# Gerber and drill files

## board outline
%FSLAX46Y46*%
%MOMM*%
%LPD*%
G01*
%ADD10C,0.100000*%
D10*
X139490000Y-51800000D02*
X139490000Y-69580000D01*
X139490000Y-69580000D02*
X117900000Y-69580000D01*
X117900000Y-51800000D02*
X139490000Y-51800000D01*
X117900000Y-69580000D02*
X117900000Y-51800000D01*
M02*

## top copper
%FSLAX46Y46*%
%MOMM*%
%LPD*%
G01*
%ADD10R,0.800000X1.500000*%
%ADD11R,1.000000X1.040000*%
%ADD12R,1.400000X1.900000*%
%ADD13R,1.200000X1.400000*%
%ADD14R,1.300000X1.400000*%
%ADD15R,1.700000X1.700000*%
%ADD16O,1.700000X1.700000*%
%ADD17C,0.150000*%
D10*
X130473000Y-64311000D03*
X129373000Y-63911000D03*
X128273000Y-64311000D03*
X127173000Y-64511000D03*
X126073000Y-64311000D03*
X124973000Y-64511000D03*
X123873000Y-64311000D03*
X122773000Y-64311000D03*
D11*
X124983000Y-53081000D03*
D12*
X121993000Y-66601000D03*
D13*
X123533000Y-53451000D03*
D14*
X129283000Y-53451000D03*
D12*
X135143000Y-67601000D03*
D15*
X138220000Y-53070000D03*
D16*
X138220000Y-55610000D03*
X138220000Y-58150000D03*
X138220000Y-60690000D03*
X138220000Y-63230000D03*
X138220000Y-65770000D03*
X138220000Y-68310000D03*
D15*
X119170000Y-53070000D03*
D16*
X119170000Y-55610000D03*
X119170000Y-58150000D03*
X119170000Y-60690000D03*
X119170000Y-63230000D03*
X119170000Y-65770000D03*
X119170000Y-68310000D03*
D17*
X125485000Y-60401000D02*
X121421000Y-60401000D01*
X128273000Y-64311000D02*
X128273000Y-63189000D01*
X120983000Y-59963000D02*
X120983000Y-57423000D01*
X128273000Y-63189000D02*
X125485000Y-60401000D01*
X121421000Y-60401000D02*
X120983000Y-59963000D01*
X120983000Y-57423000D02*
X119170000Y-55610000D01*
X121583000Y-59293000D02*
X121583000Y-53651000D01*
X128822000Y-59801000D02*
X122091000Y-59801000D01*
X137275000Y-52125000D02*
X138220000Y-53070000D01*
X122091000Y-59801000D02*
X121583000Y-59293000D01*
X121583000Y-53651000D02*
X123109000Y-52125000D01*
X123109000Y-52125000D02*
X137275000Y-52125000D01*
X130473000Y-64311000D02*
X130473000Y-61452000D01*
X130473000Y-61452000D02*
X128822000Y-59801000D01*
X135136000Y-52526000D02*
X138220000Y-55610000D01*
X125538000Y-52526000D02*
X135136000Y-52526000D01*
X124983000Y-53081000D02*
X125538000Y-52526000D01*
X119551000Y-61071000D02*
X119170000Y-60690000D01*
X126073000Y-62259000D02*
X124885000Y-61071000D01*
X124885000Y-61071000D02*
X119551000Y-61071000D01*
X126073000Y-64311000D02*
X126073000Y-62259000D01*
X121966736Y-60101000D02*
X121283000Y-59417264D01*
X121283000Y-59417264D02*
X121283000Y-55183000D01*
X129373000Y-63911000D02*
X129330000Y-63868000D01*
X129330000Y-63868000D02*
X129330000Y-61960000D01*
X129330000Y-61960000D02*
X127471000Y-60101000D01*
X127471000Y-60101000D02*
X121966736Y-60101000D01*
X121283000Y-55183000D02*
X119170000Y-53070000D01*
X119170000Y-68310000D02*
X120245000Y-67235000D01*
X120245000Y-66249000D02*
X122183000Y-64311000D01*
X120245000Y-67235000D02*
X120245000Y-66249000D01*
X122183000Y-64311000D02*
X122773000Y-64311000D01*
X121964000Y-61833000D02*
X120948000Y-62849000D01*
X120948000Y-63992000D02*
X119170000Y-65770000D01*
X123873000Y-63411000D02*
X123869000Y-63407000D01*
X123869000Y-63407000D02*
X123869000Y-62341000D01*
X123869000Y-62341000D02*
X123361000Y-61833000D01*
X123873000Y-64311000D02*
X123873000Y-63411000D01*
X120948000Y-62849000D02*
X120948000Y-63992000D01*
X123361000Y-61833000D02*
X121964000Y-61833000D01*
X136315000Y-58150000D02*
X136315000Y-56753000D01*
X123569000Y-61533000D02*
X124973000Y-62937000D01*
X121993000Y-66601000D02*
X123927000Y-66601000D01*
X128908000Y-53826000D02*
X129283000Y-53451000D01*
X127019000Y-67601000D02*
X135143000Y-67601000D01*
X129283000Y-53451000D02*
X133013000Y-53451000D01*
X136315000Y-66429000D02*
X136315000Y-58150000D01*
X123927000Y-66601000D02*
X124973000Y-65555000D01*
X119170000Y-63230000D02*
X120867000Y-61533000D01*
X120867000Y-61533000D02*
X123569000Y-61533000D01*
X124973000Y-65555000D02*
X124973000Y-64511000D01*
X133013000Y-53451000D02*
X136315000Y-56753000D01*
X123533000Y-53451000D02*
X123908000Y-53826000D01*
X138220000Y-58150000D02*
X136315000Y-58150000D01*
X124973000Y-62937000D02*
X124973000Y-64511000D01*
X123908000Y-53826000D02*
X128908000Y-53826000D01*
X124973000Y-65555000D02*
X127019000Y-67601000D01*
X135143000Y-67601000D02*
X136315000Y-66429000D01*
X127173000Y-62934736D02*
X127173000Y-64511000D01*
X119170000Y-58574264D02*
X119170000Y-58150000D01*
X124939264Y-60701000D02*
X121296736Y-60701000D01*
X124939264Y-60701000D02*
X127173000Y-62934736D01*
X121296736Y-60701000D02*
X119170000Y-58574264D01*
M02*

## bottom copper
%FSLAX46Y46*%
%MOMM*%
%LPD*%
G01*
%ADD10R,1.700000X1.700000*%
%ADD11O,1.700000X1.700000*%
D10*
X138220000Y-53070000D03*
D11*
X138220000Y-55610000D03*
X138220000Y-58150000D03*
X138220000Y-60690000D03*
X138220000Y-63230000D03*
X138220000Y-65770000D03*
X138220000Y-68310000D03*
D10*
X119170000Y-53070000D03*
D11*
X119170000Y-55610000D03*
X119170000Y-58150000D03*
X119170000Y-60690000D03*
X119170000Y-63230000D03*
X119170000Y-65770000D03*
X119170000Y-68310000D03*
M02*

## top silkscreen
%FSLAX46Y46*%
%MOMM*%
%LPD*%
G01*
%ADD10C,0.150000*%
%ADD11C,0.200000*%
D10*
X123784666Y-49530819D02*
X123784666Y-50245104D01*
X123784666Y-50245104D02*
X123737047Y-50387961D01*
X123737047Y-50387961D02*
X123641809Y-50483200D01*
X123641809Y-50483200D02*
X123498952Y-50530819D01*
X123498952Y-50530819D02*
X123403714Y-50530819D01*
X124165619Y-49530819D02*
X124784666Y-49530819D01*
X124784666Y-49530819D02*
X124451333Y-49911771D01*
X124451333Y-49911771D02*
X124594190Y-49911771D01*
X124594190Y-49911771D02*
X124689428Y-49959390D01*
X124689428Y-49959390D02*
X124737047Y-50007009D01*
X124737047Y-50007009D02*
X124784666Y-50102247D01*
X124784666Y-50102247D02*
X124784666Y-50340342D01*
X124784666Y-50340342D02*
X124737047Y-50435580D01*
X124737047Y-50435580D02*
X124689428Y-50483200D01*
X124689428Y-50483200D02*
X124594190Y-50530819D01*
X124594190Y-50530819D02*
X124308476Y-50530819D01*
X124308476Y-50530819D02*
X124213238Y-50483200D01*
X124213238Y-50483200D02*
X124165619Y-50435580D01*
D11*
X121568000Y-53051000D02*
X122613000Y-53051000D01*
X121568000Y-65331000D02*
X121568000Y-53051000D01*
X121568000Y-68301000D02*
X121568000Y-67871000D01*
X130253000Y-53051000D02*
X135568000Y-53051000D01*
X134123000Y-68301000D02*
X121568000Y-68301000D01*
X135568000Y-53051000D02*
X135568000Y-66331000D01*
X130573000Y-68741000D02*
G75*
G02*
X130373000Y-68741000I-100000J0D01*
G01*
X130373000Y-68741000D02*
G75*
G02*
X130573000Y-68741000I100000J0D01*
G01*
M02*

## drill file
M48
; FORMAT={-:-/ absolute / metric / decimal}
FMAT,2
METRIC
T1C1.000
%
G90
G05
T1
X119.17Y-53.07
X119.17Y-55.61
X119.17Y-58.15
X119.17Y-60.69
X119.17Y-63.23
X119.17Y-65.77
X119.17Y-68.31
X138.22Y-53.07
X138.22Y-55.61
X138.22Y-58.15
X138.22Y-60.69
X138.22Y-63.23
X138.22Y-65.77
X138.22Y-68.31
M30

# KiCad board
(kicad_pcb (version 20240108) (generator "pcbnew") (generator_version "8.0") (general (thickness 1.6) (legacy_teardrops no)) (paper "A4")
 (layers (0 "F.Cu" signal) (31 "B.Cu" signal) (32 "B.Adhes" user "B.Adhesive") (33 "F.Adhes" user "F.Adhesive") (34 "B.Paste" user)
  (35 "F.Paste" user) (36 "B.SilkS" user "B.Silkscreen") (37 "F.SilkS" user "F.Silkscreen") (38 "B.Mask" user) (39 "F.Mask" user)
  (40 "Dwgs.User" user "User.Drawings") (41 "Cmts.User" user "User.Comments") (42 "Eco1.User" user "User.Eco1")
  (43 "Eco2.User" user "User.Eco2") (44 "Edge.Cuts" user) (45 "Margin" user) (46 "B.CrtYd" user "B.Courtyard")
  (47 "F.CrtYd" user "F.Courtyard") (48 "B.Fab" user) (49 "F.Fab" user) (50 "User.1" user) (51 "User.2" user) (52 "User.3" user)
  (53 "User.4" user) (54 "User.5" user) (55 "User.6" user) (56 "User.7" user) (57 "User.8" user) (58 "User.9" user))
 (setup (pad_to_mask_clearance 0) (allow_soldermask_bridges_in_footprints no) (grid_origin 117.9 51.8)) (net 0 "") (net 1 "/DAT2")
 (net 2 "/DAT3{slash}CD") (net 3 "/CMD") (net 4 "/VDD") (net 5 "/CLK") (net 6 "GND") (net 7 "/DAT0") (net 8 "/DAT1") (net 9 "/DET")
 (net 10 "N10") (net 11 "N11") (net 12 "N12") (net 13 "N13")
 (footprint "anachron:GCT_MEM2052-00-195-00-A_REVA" (layer "F.Cu") (at 128.568 60.676)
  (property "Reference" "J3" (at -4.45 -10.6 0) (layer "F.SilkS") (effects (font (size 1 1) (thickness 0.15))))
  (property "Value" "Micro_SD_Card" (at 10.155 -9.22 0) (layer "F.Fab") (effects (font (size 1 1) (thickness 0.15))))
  (fp_line (start -7 -7.625) (end -5.955 -7.625) (stroke (width 0.2) (type solid)) (layer "F.SilkS"))
  (fp_line (start -7 4.655) (end -7 -7.625) (stroke (width 0.2) (type solid)) (layer "F.SilkS"))
  (fp_line (start -7 7.625) (end -7 7.195) (stroke (width 0.2) (type solid)) (layer "F.SilkS"))
  (fp_line (start 1.685 -7.625) (end 7 -7.625) (stroke (width 0.2) (type solid)) (layer "F.SilkS"))
  (fp_line (start 5.555 7.625) (end -7 7.625) (stroke (width 0.2) (type solid)) (layer "F.SilkS"))
  (fp_line (start 7 -7.625) (end 7 5.655) (stroke (width 0.2) (type solid)) (layer "F.SilkS"))
  (fp_circle (center 1.905 8.065) (end 2.005 8.065) (stroke (width 0.2) (type solid)) (fill none) (layer "F.SilkS"))
  (pad "1" smd rect (at 1.905 3.635) (size 0.8 1.5) (layers "F.Cu" "F.Paste" "F.Mask") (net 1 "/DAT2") (solder_mask_margin 0.102))
  (pad "2" smd rect (at 0.805 3.235) (size 0.8 1.5) (layers "F.Cu" "F.Paste" "F.Mask") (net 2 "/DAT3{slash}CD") (solder_mask_margin 0.102))
  (pad "3" smd rect (at -0.295 3.635) (size 0.8 1.5) (layers "F.Cu" "F.Paste" "F.Mask") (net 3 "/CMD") (solder_mask_margin 0.102))
  (pad "4" smd rect (at -1.395 3.835) (size 0.8 1.5) (layers "F.Cu" "F.Paste" "F.Mask") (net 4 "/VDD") (solder_mask_margin 0.102))
  (pad "5" smd rect (at -2.495 3.635) (size 0.8 1.5) (layers "F.Cu" "F.Paste" "F.Mask") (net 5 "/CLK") (solder_mask_margin 0.102))
  (pad "6" smd rect (at -3.595 3.835) (size 0.8 1.5) (layers "F.Cu" "F.Paste" "F.Mask") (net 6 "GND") (solder_mask_margin 0.102))
  (pad "7" smd rect (at -4.695 3.635) (size 0.8 1.5) (layers "F.Cu" "F.Paste" "F.Mask") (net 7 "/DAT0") (solder_mask_margin 0.102))
  (pad "8" smd rect (at -5.795 3.635) (size 0.8 1.5) (layers "F.Cu" "F.Paste" "F.Mask") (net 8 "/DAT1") (solder_mask_margin 0.102))
  (pad "9" smd rect (at -3.585 -7.595) (size 1 1.04) (layers "F.Cu" "F.Paste" "F.Mask") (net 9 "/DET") (solder_mask_margin 0.102))
  (pad "10" smd rect (at -6.575 5.925) (size 1.4 1.9) (layers "F.Cu" "F.Paste" "F.Mask") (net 6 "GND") (solder_mask_margin 0.102))
  (pad "10" smd rect (at -5.035 -7.225) (size 1.2 1.4) (layers "F.Cu" "F.Paste" "F.Mask") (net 6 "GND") (solder_mask_margin 0.102))
  (pad "10" smd rect (at 0.715 -7.225) (size 1.3 1.4) (layers "F.Cu" "F.Paste" "F.Mask") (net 6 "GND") (solder_mask_margin 0.102))
  (pad "10" smd rect (at 6.575 6.925) (size 1.4 1.9) (layers "F.Cu" "F.Paste" "F.Mask") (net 6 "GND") (solder_mask_margin 0.102))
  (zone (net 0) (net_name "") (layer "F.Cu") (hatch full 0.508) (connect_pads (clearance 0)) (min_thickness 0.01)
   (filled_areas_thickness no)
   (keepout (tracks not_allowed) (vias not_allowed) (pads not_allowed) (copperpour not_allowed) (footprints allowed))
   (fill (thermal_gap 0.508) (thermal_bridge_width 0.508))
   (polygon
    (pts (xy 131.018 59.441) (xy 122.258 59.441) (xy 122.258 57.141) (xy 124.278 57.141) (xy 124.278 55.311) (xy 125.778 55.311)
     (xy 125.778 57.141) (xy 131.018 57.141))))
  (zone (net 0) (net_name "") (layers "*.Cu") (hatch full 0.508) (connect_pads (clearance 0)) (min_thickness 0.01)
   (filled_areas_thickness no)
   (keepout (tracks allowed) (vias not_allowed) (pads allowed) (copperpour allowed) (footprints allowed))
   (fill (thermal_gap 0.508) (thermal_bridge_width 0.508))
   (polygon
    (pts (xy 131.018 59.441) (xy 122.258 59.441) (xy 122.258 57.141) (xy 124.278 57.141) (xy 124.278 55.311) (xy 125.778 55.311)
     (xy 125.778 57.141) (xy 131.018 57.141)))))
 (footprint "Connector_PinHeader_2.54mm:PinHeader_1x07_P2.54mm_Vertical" (layer "B.Cu") (at 138.22 53.07 180)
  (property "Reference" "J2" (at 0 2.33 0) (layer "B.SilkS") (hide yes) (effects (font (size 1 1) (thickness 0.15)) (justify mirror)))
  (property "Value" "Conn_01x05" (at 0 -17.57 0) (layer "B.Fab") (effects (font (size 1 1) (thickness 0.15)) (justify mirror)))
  (pad "1" thru_hole rect (at 0 0 180) (size 1.7 1.7) (drill 1) (layers "*.Cu" "*.Mask") (remove_unused_layers no) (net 1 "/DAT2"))
  (pad "2" thru_hole oval (at 0 -2.54 180) (size 1.7 1.7) (drill 1) (layers "*.Cu" "*.Mask") (remove_unused_layers no) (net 9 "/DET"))
  (pad "3" thru_hole oval (at 0 -5.08 180) (size 1.7 1.7) (drill 1) (layers "*.Cu" "*.Mask") (remove_unused_layers no) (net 6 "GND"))
  (pad "4" thru_hole oval (at 0 -7.62 180) (size 1.7 1.7) (drill 1) (layers "*.Cu" "*.Mask") (remove_unused_layers no) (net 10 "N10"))
  (pad "5" thru_hole oval (at 0 -10.16 180) (size 1.7 1.7) (drill 1) (layers "*.Cu" "*.Mask") (remove_unused_layers no) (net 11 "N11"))
  (pad "6" thru_hole oval (at 0 -12.7 180) (size 1.7 1.7) (drill 1) (layers "*.Cu" "*.Mask") (remove_unused_layers no) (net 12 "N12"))
  (pad "7" thru_hole oval (at 0 -15.24 180) (size 1.7 1.7) (drill 1) (layers "*.Cu" "*.Mask") (remove_unused_layers no) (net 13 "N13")))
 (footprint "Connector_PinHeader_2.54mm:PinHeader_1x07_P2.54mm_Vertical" (layer "B.Cu") (at 119.17 53.07 180)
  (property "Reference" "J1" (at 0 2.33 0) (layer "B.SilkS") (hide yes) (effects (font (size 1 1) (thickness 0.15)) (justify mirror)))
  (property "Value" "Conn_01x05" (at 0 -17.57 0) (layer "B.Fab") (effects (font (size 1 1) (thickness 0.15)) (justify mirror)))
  (pad "1" thru_hole rect (at 0 0 180) (size 1.7 1.7) (drill 1) (layers "*.Cu" "*.Mask") (remove_unused_layers no) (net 2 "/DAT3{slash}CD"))
  (pad "2" thru_hole oval (at 0 -2.54 180) (size 1.7 1.7) (drill 1) (layers "*.Cu" "*.Mask") (remove_unused_layers no) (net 3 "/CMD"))
  (pad "3" thru_hole oval (at 0 -5.08 180) (size 1.7 1.7) (drill 1) (layers "*.Cu" "*.Mask") (remove_unused_layers no) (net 4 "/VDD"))
  (pad "4" thru_hole oval (at 0 -7.62 180) (size 1.7 1.7) (drill 1) (layers "*.Cu" "*.Mask") (remove_unused_layers no) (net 5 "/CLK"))
  (pad "5" thru_hole oval (at 0 -10.16 180) (size 1.7 1.7) (drill 1) (layers "*.Cu" "*.Mask") (remove_unused_layers no) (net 6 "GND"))
  (pad "6" thru_hole oval (at 0 -12.7 180) (size 1.7 1.7) (drill 1) (layers "*.Cu" "*.Mask") (remove_unused_layers no) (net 7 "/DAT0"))
  (pad "7" thru_hole oval (at 0 -15.24 180) (size 1.7 1.7) (drill 1) (layers "*.Cu" "*.Mask") (remove_unused_layers no) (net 8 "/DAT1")))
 (gr_line (start 139.49 51.8) (end 139.49 69.58) (stroke (width 0.1) (type default)) (layer "Edge.Cuts"))
 (gr_line (start 139.49 69.58) (end 117.9 69.58) (stroke (width 0.1) (type default)) (layer "Edge.Cuts"))
 (gr_line (start 117.9 51.8) (end 139.49 51.8) (stroke (width 0.1) (type default)) (layer "Edge.Cuts"))
 (gr_line (start 117.9 69.58) (end 117.9 51.8) (stroke (width 0.1) (type default)) (layer "Edge.Cuts"))
 (segment (start 125.485 60.401) (end 121.421 60.401) (width 0.15) (layer "F.Cu") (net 3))
 (segment (start 128.273 64.311) (end 128.273 63.189) (width 0.15) (layer "F.Cu") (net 3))
 (segment (start 120.983 59.963) (end 120.983 57.423) (width 0.15) (layer "F.Cu") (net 3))
 (segment (start 128.273 63.189) (end 125.485 60.401) (width 0.15) (layer "F.Cu") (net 3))
 (segment (start 121.421 60.401) (end 120.983 59.963) (width 0.15) (layer "F.Cu") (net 3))
 (segment (start 120.983 57.423) (end 119.17 55.61) (width 0.15) (layer "F.Cu") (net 3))
 (segment (start 121.583 59.293) (end 121.583 53.651) (width 0.15) (layer "F.Cu") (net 1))
 (segment (start 128.822 59.801) (end 122.091 59.801) (width 0.15) (layer "F.Cu") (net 1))
 (segment (start 137.275 52.125) (end 138.22 53.07) (width 0.15) (layer "F.Cu") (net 1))
 (segment (start 122.091 59.801) (end 121.583 59.293) (width 0.15) (layer "F.Cu") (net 1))
 (segment (start 121.583 53.651) (end 123.109 52.125) (width 0.15) (layer "F.Cu") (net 1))
 (segment (start 123.109 52.125) (end 137.275 52.125) (width 0.15) (layer "F.Cu") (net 1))
 (segment (start 130.473 64.311) (end 130.473 61.452) (width 0.15) (layer "F.Cu") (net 1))
 (segment (start 130.473 61.452) (end 128.822 59.801) (width 0.15) (layer "F.Cu") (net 1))
 (segment (start 135.136 52.526) (end 138.22 55.61) (width 0.15) (layer "F.Cu") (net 9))
 (segment (start 125.538 52.526) (end 135.136 52.526) (width 0.15) (layer "F.Cu") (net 9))
 (segment (start 124.983 53.081) (end 125.538 52.526) (width 0.15) (layer "F.Cu") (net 9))
 (segment (start 119.551 61.071) (end 119.17 60.69) (width 0.15) (layer "F.Cu") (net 5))
 (segment (start 126.073 62.259) (end 124.885 61.071) (width 0.15) (layer "F.Cu") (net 5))
 (segment (start 124.885 61.071) (end 119.551 61.071) (width 0.15) (layer "F.Cu") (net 5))
 (segment (start 126.073 64.311) (end 126.073 62.259) (width 0.15) (layer "F.Cu") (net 5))
 (segment (start 121.966736 60.101) (end 121.283 59.417264) (width 0.15) (layer "F.Cu") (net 2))
 (segment (start 121.283 59.417264) (end 121.283 55.183) (width 0.15) (layer "F.Cu") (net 2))
 (segment (start 129.373 63.911) (end 129.33 63.868) (width 0.15) (layer "F.Cu") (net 2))
 (segment (start 129.33 63.868) (end 129.33 61.96) (width 0.15) (layer "F.Cu") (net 2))
 (segment (start 129.33 61.96) (end 127.471 60.101) (width 0.15) (layer "F.Cu") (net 2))
 (segment (start 127.471 60.101) (end 121.966736 60.101) (width 0.15) (layer "F.Cu") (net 2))
 (segment (start 121.283 55.183) (end 119.17 53.07) (width 0.15) (layer "F.Cu") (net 2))
 (segment (start 119.17 68.31) (end 120.245 67.235) (width 0.15) (layer "F.Cu") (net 8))
 (segment (start 120.245 66.249) (end 122.183 64.311) (width 0.15) (layer "F.Cu") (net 8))
 (segment (start 120.245 67.235) (end 120.245 66.249) (width 0.15) (layer "F.Cu") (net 8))
 (segment (start 122.183 64.311) (end 122.773 64.311) (width 0.15) (layer "F.Cu") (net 8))
 (segment (start 121.964 61.833) (end 120.948 62.849) (width 0.15) (layer "F.Cu") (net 7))
 (segment (start 120.948 63.992) (end 119.17 65.77) (width 0.15) (layer "F.Cu") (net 7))
 (segment (start 123.873 63.411) (end 123.869 63.407) (width 0.15) (layer "F.Cu") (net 7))
 (segment (start 123.869 63.407) (end 123.869 62.341) (width 0.15) (layer "F.Cu") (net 7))
 (segment (start 123.869 62.341) (end 123.361 61.833) (width 0.15) (layer "F.Cu") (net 7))
 (segment (start 123.873 64.311) (end 123.873 63.411) (width 0.15) (layer "F.Cu") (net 7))
 (segment (start 120.948 62.849) (end 120.948 63.992) (width 0.15) (layer "F.Cu") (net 7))
 (segment (start 123.361 61.833) (end 121.964 61.833) (width 0.15) (layer "F.Cu") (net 7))
 (segment (start 136.315 58.15) (end 136.315 56.753) (width 0.15) (layer "F.Cu") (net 6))
 (segment (start 123.569 61.533) (end 124.973 62.937) (width 0.15) (layer "F.Cu") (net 6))
 (segment (start 121.993 66.601) (end 123.927 66.601) (width 0.15) (layer "F.Cu") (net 6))
 (segment (start 128.908 53.826) (end 129.283 53.451) (width 0.15) (layer "F.Cu") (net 6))
 (segment (start 127.019 67.601) (end 135.143 67.601) (width 0.15) (layer "F.Cu") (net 6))
 (segment (start 129.283 53.451) (end 133.013 53.451) (width 0.15) (layer "F.Cu") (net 6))
 (segment (start 136.315 66.429) (end 136.315 58.15) (width 0.15) (layer "F.Cu") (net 6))
 (segment (start 123.927 66.601) (end 124.973 65.555) (width 0.15) (layer "F.Cu") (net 6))
 (segment (start 119.17 63.23) (end 120.867 61.533) (width 0.15) (layer "F.Cu") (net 6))
 (segment (start 120.867 61.533) (end 123.569 61.533) (width 0.15) (layer "F.Cu") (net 6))
 (segment (start 124.973 65.555) (end 124.973 64.511) (width 0.15) (layer "F.Cu") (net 6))
 (segment (start 133.013 53.451) (end 136.315 56.753) (width 0.15) (layer "F.Cu") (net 6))
 (segment (start 123.533 53.451) (end 123.908 53.826) (width 0.15) (layer "F.Cu") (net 6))
 (segment (start 138.22 58.15) (end 136.315 58.15) (width 0.15) (layer "F.Cu") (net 6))
 (segment (start 124.973 62.937) (end 124.973 64.511) (width 0.15) (layer "F.Cu") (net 6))
 (segment (start 123.908 53.826) (end 128.908 53.826) (width 0.15) (layer "F.Cu") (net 6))
 (segment (start 124.973 65.555) (end 127.019 67.601) (width 0.15) (layer "F.Cu") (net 6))
 (segment (start 135.143 67.601) (end 136.315 66.429) (width 0.15) (layer "F.Cu") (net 6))
 (segment (start 127.173 62.934736) (end 127.173 64.511) (width 0.15) (layer "F.Cu") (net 4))
 (segment (start 119.17 58.574264) (end 119.17 58.15) (width 0.15) (layer "F.Cu") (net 4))
 (segment (start 124.939264 60.701) (end 121.296736 60.701) (width 0.15) (layer "F.Cu") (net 4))
 (segment (start 124.939264 60.701) (end 127.173 62.934736) (width 0.15) (layer "F.Cu") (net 4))
 (segment (start 121.296736 60.701) (end 119.17 58.574264) (width 0.15) (layer "F.Cu") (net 4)))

